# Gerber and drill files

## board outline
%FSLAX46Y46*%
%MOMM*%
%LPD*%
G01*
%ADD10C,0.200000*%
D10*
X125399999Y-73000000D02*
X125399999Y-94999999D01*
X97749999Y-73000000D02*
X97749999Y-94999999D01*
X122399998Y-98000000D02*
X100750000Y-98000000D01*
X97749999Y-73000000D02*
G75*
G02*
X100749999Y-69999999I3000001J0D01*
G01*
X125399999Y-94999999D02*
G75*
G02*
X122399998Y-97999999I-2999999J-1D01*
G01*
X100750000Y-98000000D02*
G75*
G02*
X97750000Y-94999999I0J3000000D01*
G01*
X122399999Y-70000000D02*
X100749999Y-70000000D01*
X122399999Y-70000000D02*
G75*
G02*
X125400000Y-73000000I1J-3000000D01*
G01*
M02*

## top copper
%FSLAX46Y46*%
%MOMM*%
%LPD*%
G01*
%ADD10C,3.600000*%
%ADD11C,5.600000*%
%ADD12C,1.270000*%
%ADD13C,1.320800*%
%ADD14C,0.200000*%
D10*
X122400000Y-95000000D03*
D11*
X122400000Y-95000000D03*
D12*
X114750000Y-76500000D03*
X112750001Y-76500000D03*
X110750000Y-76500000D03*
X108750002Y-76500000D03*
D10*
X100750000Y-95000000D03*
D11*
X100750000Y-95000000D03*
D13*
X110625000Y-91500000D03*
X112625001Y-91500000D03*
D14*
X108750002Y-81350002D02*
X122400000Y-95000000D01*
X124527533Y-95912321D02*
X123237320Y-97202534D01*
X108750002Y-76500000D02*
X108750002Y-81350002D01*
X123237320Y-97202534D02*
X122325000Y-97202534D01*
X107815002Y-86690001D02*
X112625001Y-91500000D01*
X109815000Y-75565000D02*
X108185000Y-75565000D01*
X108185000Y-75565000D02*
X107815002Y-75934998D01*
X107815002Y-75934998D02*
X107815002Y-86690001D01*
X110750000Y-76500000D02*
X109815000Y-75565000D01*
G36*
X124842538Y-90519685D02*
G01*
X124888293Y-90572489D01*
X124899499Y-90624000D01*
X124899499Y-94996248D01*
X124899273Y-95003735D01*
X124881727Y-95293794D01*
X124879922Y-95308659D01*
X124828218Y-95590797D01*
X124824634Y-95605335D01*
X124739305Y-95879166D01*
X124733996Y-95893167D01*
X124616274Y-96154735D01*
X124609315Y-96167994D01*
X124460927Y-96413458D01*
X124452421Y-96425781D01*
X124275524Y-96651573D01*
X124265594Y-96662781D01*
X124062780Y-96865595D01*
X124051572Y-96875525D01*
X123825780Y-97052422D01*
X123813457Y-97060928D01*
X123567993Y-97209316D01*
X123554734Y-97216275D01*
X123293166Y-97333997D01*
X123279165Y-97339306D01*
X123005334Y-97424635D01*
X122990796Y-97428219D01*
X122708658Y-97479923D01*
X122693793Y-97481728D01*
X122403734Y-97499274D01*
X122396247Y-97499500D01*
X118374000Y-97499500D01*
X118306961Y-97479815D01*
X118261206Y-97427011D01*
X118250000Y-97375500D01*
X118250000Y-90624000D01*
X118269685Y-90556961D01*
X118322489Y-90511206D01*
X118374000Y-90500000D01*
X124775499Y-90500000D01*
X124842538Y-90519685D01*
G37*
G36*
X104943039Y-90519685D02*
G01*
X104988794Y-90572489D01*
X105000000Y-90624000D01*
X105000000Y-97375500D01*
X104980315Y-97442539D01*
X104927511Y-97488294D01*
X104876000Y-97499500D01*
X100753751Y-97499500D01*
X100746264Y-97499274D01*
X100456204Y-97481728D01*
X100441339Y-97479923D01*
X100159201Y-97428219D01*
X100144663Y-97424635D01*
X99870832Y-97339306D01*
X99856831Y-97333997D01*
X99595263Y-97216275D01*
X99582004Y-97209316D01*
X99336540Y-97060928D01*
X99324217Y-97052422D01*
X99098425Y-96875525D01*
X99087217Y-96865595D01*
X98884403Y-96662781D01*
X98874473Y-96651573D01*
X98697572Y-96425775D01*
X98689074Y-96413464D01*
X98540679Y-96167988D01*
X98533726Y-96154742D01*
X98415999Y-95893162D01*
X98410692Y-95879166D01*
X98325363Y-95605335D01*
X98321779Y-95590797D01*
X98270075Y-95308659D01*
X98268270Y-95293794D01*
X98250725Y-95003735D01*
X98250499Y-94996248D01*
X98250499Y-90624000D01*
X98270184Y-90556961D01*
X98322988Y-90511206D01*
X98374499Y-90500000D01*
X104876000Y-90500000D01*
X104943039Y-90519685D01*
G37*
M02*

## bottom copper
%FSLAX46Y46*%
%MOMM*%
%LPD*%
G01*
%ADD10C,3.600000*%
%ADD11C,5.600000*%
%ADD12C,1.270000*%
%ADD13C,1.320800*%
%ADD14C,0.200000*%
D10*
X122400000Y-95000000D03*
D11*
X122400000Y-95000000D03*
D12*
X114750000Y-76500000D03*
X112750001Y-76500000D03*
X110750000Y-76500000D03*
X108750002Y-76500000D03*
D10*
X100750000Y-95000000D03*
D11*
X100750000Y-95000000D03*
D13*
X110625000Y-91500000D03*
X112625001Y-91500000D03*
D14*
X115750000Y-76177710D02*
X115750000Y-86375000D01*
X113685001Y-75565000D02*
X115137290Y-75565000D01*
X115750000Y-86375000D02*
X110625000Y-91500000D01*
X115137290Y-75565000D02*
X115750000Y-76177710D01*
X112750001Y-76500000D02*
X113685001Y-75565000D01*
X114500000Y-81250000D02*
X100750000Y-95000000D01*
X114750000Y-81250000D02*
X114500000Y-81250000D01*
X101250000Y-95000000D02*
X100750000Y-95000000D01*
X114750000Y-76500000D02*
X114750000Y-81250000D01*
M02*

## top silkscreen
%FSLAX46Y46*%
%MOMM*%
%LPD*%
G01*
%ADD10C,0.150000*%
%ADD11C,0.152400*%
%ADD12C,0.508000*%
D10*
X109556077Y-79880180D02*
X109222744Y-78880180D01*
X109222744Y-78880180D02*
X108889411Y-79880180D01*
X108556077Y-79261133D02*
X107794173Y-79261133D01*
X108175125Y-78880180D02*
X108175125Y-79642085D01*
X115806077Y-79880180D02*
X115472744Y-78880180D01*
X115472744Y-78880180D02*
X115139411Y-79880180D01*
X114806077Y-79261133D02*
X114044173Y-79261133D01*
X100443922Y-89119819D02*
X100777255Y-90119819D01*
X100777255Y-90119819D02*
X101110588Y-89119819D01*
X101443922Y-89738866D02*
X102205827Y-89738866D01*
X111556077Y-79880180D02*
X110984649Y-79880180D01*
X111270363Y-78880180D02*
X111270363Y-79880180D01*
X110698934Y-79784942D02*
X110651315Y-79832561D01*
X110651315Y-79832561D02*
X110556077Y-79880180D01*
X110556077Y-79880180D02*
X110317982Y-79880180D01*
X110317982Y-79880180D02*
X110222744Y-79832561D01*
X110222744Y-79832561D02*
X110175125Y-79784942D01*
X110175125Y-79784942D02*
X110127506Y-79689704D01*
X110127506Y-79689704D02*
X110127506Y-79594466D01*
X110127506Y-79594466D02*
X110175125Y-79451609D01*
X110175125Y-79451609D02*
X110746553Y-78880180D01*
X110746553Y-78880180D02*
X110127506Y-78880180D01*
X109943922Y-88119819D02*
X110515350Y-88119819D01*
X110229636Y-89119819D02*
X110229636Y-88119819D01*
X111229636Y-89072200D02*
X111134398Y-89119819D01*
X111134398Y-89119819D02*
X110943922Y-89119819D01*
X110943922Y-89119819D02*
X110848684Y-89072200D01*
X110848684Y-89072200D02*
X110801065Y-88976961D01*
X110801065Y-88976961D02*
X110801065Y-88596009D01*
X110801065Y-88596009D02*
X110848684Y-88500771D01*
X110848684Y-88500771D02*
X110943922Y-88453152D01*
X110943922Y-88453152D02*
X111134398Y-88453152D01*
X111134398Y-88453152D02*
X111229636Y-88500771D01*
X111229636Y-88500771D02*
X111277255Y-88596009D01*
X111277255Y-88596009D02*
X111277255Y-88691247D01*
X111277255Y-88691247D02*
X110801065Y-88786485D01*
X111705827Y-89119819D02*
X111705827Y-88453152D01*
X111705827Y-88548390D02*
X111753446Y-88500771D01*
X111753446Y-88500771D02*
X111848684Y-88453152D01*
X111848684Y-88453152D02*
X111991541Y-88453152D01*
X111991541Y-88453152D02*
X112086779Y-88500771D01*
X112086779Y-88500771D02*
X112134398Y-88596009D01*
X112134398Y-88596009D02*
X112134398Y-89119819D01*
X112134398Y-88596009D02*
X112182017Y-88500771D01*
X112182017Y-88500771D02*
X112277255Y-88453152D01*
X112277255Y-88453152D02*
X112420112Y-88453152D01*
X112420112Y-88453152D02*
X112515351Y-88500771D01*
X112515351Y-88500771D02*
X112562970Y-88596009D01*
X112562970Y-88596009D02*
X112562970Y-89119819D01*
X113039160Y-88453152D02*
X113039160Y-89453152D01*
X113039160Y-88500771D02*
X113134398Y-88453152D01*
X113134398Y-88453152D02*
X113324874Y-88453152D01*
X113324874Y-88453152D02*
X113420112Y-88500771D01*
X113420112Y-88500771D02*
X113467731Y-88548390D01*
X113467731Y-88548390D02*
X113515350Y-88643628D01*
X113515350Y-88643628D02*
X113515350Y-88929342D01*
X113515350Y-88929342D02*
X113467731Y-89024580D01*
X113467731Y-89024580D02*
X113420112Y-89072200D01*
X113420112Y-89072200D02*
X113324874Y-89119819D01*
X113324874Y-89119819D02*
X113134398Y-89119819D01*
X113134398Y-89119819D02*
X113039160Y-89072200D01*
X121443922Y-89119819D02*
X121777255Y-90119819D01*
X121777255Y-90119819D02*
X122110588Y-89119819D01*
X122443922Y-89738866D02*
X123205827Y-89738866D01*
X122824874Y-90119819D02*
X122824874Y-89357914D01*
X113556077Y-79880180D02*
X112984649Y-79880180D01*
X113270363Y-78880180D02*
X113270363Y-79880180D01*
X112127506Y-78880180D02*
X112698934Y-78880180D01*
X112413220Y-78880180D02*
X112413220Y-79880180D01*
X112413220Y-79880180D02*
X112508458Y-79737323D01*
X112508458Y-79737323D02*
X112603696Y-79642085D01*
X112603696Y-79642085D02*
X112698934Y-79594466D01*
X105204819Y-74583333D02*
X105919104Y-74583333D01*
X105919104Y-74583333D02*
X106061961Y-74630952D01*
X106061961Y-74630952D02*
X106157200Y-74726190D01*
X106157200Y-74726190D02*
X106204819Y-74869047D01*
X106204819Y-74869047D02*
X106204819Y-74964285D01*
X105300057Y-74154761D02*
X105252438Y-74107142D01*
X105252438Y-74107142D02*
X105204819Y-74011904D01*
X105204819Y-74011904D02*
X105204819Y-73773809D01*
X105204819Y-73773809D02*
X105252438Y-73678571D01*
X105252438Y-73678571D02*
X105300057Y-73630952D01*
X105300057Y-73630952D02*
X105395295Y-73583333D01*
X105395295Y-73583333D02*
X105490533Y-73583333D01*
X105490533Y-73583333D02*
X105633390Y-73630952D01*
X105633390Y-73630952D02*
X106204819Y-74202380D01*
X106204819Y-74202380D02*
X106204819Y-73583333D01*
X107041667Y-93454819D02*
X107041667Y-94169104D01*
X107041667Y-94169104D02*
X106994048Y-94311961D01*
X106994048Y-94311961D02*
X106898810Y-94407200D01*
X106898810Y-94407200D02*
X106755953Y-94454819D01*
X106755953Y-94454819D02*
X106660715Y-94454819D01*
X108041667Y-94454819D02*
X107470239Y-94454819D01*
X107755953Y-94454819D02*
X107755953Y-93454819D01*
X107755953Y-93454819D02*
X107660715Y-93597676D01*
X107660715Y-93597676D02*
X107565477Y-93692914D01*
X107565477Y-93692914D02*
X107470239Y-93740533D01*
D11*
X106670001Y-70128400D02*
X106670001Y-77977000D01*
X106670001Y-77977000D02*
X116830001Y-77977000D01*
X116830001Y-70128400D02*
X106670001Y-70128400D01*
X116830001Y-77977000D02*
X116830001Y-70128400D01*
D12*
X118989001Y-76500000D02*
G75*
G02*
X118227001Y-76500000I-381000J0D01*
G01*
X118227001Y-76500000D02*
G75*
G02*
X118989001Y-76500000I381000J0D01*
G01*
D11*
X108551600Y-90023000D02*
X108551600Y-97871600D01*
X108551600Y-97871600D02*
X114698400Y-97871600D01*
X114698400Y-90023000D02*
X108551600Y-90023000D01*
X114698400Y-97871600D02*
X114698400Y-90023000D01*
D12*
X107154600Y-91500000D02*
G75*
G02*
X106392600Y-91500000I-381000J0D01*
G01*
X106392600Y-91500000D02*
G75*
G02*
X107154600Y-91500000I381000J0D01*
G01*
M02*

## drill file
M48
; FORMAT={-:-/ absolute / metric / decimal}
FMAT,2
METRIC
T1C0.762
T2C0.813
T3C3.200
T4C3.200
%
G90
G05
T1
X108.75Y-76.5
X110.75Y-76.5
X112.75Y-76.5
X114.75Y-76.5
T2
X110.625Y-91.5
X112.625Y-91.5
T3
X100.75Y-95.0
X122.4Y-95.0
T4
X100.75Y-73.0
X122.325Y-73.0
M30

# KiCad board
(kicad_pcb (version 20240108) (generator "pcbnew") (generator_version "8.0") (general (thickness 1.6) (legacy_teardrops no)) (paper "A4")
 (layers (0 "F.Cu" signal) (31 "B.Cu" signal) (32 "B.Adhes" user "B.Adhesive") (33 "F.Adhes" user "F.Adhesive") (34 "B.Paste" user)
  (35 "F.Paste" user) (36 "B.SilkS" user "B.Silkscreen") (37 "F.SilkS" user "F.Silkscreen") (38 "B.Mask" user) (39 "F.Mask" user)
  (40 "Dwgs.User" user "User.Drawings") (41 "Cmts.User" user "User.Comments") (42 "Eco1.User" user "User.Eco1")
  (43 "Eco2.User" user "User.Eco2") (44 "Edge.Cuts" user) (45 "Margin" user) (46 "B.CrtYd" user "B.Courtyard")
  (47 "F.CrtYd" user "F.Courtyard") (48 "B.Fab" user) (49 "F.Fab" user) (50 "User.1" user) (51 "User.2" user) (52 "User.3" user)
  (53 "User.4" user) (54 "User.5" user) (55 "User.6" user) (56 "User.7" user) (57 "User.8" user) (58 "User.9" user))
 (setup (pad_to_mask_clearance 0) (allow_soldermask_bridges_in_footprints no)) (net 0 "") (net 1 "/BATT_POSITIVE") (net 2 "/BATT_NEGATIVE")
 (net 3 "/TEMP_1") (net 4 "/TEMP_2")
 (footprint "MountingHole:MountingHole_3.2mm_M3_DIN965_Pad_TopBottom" (layer "F.Cu") (at 122.4 95)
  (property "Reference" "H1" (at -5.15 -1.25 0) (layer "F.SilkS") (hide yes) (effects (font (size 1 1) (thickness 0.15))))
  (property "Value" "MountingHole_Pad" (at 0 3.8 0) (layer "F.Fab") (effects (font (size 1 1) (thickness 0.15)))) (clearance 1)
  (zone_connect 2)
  (pad "1" thru_hole circle (at 0 0) (size 3.6 3.6) (drill 3.2) (layers "*.Cu" "*.Mask") (remove_unused_layers no) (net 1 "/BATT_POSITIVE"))
  (pad "1" connect circle (at 0 0) (size 5.6 5.6) (layers "F.Cu" "F.Mask") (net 1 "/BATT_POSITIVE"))
  (pad "1" connect circle (at 0 0) (size 5.6 5.6) (layers "B.Cu" "B.Mask") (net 1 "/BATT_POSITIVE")))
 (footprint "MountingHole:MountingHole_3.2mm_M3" (layer "F.Cu") (at 122.324999 73)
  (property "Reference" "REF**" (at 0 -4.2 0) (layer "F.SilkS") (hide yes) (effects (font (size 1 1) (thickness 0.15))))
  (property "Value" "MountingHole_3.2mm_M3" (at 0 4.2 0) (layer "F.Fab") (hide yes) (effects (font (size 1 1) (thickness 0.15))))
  (pad "" np_thru_hole circle (at 0 0) (size 3.2 3.2) (drill 3.2) (layers "F&B.Cu" "*.Mask")))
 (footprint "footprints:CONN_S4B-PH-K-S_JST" (layer "F.Cu") (at 114.75 76.5 180)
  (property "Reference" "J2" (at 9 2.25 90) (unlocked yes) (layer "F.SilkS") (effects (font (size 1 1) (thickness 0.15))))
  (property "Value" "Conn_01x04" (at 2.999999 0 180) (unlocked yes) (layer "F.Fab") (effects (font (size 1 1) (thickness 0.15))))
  (fp_line (start 8.079999 6.3716) (end 8.079999 -1.477) (stroke (width 0.1524) (type solid)) (layer "F.SilkS"))
  (fp_line (start 8.079999 -1.477) (end -2.080001 -1.477) (stroke (width 0.1524) (type solid)) (layer "F.SilkS"))
  (fp_line (start -2.080001 6.3716) (end 8.079999 6.3716) (stroke (width 0.1524) (type solid)) (layer "F.SilkS"))
  (fp_line (start -2.080001 -1.477) (end -2.080001 6.3716) (stroke (width 0.1524) (type solid)) (layer "F.SilkS"))
  (fp_circle (center -3.858001 0) (end -3.477001 0) (stroke (width 0.508) (type solid)) (fill none) (layer "F.SilkS"))
  (pad "1" thru_hole circle (at 0 0 180) (size 1.27 1.27) (drill 0.762) (layers "*.Cu" "*.Mask") (remove_unused_layers no)
   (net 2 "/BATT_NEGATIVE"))
  (pad "2" thru_hole circle (at 1.999999 0 180) (size 1.27 1.27) (drill 0.762) (layers "*.Cu" "*.Mask") (remove_unused_layers no)
   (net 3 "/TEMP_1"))
  (pad "3" thru_hole circle (at 4 0 180) (size 1.27 1.27) (drill 0.762) (layers "*.Cu" "*.Mask") (remove_unused_layers no) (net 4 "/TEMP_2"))
  (pad "4" thru_hole circle (at 5.999998 0 180) (size 1.27 1.27) (drill 0.762) (layers "*.Cu" "*.Mask") (remove_unused_layers no)
   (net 1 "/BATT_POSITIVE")))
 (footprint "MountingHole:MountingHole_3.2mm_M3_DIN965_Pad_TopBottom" (layer "F.Cu") (at 100.75 95)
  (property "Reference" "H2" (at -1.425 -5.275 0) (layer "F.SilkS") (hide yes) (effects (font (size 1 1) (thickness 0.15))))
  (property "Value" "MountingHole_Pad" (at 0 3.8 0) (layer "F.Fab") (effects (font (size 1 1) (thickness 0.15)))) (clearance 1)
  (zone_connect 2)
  (pad "1" thru_hole circle (at 0 0) (size 3.6 3.6) (drill 3.2) (layers "*.Cu" "*.Mask") (remove_unused_layers no) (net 2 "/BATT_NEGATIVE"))
  (pad "1" connect circle (at 0 0) (size 5.6 5.6) (layers "F.Cu" "F.Mask") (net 2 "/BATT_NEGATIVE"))
  (pad "1" connect circle (at 0 0) (size 5.6 5.6) (layers "B.Cu" "B.Mask") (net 2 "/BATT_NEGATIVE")))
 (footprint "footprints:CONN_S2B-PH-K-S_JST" (layer "F.Cu") (at 110.625 91.5)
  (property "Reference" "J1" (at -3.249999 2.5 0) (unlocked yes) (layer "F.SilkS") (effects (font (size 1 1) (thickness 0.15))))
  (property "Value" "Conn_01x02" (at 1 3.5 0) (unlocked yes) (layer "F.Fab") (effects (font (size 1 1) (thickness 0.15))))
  (fp_line (start -2.0734 -1.477) (end -2.0734 6.3716) (stroke (width 0.1524) (type solid)) (layer "F.SilkS"))
  (fp_line (start -2.0734 6.3716) (end 4.0734 6.3716) (stroke (width 0.1524) (type solid)) (layer "F.SilkS"))
  (fp_line (start 4.0734 -1.477) (end -2.0734 -1.477) (stroke (width 0.1524) (type solid)) (layer "F.SilkS"))
  (fp_line (start 4.0734 6.3716) (end 4.0734 -1.477) (stroke (width 0.1524) (type solid)) (layer "F.SilkS"))
  (fp_circle (center -3.8514 0) (end -3.4704 0) (stroke (width 0.508) (type solid)) (fill none) (layer "F.SilkS"))
  (pad "1" thru_hole circle (at 0 0) (size 1.3208 1.3208) (drill 0.8128) (layers "*.Cu" "*.Mask") (remove_unused_layers no)
   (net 3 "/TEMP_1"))
  (pad "2" thru_hole circle (at 2.000001 0) (size 1.3208 1.3208) (drill 0.8128) (layers "*.Cu" "*.Mask") (remove_unused_layers no)
   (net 4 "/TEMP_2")))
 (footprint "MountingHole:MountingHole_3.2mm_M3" (layer "F.Cu") (at 100.75 73)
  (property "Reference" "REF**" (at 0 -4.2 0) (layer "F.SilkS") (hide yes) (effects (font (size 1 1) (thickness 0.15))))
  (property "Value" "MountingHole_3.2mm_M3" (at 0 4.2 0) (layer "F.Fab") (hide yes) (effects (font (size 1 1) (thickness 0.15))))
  (pad "" np_thru_hole circle (at 0 0) (size 3.2 3.2) (drill 3.2) (layers "*.Cu" "*.Mask")))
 (gr_line (start 125.399999 73) (end 125.399999 94.999999) (stroke (width 0.2) (type default)) (layer "Edge.Cuts"))
 (gr_line (start 97.749999 73) (end 97.749999 94.999999) (stroke (width 0.2) (type default)) (layer "Edge.Cuts"))
 (gr_line (start 122.399998 98) (end 100.75 98) (stroke (width 0.2) (type default)) (layer "Edge.Cuts"))
 (gr_arc (start 97.749999 73) (mid 98.628679 70.87868) (end 100.749999 70) (stroke (width 0.2) (type default)) (layer "Edge.Cuts"))
 (gr_arc (start 125.399999 94.999999) (mid 124.521319 97.12132) (end 122.399998 98) (stroke (width 0.2) (type default)) (layer "Edge.Cuts"))
 (gr_arc (start 100.75 98) (mid 98.628679 97.12132) (end 97.749999 94.999999) (stroke (width 0.2) (type default)) (layer "Edge.Cuts"))
 (gr_line (start 122.399999 70) (end 100.749999 70) (stroke (width 0.2) (type default)) (layer "Edge.Cuts"))
 (gr_arc (start 122.399999 70) (mid 124.521319 70.87868) (end 125.399999 73) (stroke (width 0.2) (type default)) (layer "Edge.Cuts"))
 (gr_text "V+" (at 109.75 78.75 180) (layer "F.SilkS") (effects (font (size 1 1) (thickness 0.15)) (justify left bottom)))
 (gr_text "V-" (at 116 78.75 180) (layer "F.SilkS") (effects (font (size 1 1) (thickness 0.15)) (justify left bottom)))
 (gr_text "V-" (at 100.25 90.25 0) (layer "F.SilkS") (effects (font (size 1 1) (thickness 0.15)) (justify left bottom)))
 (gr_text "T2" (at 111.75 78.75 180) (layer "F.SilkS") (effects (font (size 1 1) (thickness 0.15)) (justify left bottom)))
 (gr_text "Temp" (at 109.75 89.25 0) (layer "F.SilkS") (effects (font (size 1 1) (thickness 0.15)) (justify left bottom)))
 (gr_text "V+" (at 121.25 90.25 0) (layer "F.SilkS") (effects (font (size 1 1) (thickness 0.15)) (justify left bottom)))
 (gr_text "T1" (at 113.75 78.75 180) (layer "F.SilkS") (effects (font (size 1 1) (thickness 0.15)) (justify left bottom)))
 (segment (start 115.75 76.17771) (end 115.75 86.375) (width 0.2) (layer "B.Cu") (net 3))
 (segment (start 113.685001 75.565) (end 115.13729 75.565) (width 0.2) (layer "B.Cu") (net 3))
 (segment (start 115.75 86.375) (end 110.625 91.5) (width 0.2) (layer "B.Cu") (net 3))
 (segment (start 115.13729 75.565) (end 115.75 76.17771) (width 0.2) (layer "B.Cu") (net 3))
 (segment (start 112.750001 76.5) (end 113.685001 75.565) (width 0.2) (layer "B.Cu") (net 3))
 (segment (start 108.750002 81.350002) (end 122.4 95) (width 0.2) (layer "F.Cu") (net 1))
 (segment (start 124.527533 95.912321) (end 123.23732 97.202534) (width 0.2) (layer "F.Cu") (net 1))
 (segment (start 108.750002 76.5) (end 108.750002 81.350002) (width 0.2) (layer "F.Cu") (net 1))
 (segment (start 123.23732 97.202534) (end 122.325 97.202534) (width 0.2) (layer "F.Cu") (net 1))
 (segment (start 114.5 81.25) (end 100.75 95) (width 0.2) (layer "B.Cu") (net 2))
 (segment (start 114.75 81.25) (end 114.5 81.25) (width 0.2) (layer "B.Cu") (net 2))
 (segment (start 101.25 95) (end 100.75 95) (width 0.2) (layer "B.Cu") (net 2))
 (segment (start 114.75 76.5) (end 114.75 81.25) (width 0.2) (layer "B.Cu") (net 2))
 (segment (start 107.815002 86.690001) (end 112.625001 91.5) (width 0.2) (layer "F.Cu") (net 4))
 (segment (start 109.815 75.565) (end 108.185 75.565) (width 0.2) (layer "F.Cu") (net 4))
 (segment (start 108.185 75.565) (end 107.815002 75.934998) (width 0.2) (layer "F.Cu") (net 4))
 (segment (start 107.815002 75.934998) (end 107.815002 86.690001) (width 0.2) (layer "F.Cu") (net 4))
 (segment (start 110.75 76.5) (end 109.815 75.565) (width 0.2) (layer "F.Cu") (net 4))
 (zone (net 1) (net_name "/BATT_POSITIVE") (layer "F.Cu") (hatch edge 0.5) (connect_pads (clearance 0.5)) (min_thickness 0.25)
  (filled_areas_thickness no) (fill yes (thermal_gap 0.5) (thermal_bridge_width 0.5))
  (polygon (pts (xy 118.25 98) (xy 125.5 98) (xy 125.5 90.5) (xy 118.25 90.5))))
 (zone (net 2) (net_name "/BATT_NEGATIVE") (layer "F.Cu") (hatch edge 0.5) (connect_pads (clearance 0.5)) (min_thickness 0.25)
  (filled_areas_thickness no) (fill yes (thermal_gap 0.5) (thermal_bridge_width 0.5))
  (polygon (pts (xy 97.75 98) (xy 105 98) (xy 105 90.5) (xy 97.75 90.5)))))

